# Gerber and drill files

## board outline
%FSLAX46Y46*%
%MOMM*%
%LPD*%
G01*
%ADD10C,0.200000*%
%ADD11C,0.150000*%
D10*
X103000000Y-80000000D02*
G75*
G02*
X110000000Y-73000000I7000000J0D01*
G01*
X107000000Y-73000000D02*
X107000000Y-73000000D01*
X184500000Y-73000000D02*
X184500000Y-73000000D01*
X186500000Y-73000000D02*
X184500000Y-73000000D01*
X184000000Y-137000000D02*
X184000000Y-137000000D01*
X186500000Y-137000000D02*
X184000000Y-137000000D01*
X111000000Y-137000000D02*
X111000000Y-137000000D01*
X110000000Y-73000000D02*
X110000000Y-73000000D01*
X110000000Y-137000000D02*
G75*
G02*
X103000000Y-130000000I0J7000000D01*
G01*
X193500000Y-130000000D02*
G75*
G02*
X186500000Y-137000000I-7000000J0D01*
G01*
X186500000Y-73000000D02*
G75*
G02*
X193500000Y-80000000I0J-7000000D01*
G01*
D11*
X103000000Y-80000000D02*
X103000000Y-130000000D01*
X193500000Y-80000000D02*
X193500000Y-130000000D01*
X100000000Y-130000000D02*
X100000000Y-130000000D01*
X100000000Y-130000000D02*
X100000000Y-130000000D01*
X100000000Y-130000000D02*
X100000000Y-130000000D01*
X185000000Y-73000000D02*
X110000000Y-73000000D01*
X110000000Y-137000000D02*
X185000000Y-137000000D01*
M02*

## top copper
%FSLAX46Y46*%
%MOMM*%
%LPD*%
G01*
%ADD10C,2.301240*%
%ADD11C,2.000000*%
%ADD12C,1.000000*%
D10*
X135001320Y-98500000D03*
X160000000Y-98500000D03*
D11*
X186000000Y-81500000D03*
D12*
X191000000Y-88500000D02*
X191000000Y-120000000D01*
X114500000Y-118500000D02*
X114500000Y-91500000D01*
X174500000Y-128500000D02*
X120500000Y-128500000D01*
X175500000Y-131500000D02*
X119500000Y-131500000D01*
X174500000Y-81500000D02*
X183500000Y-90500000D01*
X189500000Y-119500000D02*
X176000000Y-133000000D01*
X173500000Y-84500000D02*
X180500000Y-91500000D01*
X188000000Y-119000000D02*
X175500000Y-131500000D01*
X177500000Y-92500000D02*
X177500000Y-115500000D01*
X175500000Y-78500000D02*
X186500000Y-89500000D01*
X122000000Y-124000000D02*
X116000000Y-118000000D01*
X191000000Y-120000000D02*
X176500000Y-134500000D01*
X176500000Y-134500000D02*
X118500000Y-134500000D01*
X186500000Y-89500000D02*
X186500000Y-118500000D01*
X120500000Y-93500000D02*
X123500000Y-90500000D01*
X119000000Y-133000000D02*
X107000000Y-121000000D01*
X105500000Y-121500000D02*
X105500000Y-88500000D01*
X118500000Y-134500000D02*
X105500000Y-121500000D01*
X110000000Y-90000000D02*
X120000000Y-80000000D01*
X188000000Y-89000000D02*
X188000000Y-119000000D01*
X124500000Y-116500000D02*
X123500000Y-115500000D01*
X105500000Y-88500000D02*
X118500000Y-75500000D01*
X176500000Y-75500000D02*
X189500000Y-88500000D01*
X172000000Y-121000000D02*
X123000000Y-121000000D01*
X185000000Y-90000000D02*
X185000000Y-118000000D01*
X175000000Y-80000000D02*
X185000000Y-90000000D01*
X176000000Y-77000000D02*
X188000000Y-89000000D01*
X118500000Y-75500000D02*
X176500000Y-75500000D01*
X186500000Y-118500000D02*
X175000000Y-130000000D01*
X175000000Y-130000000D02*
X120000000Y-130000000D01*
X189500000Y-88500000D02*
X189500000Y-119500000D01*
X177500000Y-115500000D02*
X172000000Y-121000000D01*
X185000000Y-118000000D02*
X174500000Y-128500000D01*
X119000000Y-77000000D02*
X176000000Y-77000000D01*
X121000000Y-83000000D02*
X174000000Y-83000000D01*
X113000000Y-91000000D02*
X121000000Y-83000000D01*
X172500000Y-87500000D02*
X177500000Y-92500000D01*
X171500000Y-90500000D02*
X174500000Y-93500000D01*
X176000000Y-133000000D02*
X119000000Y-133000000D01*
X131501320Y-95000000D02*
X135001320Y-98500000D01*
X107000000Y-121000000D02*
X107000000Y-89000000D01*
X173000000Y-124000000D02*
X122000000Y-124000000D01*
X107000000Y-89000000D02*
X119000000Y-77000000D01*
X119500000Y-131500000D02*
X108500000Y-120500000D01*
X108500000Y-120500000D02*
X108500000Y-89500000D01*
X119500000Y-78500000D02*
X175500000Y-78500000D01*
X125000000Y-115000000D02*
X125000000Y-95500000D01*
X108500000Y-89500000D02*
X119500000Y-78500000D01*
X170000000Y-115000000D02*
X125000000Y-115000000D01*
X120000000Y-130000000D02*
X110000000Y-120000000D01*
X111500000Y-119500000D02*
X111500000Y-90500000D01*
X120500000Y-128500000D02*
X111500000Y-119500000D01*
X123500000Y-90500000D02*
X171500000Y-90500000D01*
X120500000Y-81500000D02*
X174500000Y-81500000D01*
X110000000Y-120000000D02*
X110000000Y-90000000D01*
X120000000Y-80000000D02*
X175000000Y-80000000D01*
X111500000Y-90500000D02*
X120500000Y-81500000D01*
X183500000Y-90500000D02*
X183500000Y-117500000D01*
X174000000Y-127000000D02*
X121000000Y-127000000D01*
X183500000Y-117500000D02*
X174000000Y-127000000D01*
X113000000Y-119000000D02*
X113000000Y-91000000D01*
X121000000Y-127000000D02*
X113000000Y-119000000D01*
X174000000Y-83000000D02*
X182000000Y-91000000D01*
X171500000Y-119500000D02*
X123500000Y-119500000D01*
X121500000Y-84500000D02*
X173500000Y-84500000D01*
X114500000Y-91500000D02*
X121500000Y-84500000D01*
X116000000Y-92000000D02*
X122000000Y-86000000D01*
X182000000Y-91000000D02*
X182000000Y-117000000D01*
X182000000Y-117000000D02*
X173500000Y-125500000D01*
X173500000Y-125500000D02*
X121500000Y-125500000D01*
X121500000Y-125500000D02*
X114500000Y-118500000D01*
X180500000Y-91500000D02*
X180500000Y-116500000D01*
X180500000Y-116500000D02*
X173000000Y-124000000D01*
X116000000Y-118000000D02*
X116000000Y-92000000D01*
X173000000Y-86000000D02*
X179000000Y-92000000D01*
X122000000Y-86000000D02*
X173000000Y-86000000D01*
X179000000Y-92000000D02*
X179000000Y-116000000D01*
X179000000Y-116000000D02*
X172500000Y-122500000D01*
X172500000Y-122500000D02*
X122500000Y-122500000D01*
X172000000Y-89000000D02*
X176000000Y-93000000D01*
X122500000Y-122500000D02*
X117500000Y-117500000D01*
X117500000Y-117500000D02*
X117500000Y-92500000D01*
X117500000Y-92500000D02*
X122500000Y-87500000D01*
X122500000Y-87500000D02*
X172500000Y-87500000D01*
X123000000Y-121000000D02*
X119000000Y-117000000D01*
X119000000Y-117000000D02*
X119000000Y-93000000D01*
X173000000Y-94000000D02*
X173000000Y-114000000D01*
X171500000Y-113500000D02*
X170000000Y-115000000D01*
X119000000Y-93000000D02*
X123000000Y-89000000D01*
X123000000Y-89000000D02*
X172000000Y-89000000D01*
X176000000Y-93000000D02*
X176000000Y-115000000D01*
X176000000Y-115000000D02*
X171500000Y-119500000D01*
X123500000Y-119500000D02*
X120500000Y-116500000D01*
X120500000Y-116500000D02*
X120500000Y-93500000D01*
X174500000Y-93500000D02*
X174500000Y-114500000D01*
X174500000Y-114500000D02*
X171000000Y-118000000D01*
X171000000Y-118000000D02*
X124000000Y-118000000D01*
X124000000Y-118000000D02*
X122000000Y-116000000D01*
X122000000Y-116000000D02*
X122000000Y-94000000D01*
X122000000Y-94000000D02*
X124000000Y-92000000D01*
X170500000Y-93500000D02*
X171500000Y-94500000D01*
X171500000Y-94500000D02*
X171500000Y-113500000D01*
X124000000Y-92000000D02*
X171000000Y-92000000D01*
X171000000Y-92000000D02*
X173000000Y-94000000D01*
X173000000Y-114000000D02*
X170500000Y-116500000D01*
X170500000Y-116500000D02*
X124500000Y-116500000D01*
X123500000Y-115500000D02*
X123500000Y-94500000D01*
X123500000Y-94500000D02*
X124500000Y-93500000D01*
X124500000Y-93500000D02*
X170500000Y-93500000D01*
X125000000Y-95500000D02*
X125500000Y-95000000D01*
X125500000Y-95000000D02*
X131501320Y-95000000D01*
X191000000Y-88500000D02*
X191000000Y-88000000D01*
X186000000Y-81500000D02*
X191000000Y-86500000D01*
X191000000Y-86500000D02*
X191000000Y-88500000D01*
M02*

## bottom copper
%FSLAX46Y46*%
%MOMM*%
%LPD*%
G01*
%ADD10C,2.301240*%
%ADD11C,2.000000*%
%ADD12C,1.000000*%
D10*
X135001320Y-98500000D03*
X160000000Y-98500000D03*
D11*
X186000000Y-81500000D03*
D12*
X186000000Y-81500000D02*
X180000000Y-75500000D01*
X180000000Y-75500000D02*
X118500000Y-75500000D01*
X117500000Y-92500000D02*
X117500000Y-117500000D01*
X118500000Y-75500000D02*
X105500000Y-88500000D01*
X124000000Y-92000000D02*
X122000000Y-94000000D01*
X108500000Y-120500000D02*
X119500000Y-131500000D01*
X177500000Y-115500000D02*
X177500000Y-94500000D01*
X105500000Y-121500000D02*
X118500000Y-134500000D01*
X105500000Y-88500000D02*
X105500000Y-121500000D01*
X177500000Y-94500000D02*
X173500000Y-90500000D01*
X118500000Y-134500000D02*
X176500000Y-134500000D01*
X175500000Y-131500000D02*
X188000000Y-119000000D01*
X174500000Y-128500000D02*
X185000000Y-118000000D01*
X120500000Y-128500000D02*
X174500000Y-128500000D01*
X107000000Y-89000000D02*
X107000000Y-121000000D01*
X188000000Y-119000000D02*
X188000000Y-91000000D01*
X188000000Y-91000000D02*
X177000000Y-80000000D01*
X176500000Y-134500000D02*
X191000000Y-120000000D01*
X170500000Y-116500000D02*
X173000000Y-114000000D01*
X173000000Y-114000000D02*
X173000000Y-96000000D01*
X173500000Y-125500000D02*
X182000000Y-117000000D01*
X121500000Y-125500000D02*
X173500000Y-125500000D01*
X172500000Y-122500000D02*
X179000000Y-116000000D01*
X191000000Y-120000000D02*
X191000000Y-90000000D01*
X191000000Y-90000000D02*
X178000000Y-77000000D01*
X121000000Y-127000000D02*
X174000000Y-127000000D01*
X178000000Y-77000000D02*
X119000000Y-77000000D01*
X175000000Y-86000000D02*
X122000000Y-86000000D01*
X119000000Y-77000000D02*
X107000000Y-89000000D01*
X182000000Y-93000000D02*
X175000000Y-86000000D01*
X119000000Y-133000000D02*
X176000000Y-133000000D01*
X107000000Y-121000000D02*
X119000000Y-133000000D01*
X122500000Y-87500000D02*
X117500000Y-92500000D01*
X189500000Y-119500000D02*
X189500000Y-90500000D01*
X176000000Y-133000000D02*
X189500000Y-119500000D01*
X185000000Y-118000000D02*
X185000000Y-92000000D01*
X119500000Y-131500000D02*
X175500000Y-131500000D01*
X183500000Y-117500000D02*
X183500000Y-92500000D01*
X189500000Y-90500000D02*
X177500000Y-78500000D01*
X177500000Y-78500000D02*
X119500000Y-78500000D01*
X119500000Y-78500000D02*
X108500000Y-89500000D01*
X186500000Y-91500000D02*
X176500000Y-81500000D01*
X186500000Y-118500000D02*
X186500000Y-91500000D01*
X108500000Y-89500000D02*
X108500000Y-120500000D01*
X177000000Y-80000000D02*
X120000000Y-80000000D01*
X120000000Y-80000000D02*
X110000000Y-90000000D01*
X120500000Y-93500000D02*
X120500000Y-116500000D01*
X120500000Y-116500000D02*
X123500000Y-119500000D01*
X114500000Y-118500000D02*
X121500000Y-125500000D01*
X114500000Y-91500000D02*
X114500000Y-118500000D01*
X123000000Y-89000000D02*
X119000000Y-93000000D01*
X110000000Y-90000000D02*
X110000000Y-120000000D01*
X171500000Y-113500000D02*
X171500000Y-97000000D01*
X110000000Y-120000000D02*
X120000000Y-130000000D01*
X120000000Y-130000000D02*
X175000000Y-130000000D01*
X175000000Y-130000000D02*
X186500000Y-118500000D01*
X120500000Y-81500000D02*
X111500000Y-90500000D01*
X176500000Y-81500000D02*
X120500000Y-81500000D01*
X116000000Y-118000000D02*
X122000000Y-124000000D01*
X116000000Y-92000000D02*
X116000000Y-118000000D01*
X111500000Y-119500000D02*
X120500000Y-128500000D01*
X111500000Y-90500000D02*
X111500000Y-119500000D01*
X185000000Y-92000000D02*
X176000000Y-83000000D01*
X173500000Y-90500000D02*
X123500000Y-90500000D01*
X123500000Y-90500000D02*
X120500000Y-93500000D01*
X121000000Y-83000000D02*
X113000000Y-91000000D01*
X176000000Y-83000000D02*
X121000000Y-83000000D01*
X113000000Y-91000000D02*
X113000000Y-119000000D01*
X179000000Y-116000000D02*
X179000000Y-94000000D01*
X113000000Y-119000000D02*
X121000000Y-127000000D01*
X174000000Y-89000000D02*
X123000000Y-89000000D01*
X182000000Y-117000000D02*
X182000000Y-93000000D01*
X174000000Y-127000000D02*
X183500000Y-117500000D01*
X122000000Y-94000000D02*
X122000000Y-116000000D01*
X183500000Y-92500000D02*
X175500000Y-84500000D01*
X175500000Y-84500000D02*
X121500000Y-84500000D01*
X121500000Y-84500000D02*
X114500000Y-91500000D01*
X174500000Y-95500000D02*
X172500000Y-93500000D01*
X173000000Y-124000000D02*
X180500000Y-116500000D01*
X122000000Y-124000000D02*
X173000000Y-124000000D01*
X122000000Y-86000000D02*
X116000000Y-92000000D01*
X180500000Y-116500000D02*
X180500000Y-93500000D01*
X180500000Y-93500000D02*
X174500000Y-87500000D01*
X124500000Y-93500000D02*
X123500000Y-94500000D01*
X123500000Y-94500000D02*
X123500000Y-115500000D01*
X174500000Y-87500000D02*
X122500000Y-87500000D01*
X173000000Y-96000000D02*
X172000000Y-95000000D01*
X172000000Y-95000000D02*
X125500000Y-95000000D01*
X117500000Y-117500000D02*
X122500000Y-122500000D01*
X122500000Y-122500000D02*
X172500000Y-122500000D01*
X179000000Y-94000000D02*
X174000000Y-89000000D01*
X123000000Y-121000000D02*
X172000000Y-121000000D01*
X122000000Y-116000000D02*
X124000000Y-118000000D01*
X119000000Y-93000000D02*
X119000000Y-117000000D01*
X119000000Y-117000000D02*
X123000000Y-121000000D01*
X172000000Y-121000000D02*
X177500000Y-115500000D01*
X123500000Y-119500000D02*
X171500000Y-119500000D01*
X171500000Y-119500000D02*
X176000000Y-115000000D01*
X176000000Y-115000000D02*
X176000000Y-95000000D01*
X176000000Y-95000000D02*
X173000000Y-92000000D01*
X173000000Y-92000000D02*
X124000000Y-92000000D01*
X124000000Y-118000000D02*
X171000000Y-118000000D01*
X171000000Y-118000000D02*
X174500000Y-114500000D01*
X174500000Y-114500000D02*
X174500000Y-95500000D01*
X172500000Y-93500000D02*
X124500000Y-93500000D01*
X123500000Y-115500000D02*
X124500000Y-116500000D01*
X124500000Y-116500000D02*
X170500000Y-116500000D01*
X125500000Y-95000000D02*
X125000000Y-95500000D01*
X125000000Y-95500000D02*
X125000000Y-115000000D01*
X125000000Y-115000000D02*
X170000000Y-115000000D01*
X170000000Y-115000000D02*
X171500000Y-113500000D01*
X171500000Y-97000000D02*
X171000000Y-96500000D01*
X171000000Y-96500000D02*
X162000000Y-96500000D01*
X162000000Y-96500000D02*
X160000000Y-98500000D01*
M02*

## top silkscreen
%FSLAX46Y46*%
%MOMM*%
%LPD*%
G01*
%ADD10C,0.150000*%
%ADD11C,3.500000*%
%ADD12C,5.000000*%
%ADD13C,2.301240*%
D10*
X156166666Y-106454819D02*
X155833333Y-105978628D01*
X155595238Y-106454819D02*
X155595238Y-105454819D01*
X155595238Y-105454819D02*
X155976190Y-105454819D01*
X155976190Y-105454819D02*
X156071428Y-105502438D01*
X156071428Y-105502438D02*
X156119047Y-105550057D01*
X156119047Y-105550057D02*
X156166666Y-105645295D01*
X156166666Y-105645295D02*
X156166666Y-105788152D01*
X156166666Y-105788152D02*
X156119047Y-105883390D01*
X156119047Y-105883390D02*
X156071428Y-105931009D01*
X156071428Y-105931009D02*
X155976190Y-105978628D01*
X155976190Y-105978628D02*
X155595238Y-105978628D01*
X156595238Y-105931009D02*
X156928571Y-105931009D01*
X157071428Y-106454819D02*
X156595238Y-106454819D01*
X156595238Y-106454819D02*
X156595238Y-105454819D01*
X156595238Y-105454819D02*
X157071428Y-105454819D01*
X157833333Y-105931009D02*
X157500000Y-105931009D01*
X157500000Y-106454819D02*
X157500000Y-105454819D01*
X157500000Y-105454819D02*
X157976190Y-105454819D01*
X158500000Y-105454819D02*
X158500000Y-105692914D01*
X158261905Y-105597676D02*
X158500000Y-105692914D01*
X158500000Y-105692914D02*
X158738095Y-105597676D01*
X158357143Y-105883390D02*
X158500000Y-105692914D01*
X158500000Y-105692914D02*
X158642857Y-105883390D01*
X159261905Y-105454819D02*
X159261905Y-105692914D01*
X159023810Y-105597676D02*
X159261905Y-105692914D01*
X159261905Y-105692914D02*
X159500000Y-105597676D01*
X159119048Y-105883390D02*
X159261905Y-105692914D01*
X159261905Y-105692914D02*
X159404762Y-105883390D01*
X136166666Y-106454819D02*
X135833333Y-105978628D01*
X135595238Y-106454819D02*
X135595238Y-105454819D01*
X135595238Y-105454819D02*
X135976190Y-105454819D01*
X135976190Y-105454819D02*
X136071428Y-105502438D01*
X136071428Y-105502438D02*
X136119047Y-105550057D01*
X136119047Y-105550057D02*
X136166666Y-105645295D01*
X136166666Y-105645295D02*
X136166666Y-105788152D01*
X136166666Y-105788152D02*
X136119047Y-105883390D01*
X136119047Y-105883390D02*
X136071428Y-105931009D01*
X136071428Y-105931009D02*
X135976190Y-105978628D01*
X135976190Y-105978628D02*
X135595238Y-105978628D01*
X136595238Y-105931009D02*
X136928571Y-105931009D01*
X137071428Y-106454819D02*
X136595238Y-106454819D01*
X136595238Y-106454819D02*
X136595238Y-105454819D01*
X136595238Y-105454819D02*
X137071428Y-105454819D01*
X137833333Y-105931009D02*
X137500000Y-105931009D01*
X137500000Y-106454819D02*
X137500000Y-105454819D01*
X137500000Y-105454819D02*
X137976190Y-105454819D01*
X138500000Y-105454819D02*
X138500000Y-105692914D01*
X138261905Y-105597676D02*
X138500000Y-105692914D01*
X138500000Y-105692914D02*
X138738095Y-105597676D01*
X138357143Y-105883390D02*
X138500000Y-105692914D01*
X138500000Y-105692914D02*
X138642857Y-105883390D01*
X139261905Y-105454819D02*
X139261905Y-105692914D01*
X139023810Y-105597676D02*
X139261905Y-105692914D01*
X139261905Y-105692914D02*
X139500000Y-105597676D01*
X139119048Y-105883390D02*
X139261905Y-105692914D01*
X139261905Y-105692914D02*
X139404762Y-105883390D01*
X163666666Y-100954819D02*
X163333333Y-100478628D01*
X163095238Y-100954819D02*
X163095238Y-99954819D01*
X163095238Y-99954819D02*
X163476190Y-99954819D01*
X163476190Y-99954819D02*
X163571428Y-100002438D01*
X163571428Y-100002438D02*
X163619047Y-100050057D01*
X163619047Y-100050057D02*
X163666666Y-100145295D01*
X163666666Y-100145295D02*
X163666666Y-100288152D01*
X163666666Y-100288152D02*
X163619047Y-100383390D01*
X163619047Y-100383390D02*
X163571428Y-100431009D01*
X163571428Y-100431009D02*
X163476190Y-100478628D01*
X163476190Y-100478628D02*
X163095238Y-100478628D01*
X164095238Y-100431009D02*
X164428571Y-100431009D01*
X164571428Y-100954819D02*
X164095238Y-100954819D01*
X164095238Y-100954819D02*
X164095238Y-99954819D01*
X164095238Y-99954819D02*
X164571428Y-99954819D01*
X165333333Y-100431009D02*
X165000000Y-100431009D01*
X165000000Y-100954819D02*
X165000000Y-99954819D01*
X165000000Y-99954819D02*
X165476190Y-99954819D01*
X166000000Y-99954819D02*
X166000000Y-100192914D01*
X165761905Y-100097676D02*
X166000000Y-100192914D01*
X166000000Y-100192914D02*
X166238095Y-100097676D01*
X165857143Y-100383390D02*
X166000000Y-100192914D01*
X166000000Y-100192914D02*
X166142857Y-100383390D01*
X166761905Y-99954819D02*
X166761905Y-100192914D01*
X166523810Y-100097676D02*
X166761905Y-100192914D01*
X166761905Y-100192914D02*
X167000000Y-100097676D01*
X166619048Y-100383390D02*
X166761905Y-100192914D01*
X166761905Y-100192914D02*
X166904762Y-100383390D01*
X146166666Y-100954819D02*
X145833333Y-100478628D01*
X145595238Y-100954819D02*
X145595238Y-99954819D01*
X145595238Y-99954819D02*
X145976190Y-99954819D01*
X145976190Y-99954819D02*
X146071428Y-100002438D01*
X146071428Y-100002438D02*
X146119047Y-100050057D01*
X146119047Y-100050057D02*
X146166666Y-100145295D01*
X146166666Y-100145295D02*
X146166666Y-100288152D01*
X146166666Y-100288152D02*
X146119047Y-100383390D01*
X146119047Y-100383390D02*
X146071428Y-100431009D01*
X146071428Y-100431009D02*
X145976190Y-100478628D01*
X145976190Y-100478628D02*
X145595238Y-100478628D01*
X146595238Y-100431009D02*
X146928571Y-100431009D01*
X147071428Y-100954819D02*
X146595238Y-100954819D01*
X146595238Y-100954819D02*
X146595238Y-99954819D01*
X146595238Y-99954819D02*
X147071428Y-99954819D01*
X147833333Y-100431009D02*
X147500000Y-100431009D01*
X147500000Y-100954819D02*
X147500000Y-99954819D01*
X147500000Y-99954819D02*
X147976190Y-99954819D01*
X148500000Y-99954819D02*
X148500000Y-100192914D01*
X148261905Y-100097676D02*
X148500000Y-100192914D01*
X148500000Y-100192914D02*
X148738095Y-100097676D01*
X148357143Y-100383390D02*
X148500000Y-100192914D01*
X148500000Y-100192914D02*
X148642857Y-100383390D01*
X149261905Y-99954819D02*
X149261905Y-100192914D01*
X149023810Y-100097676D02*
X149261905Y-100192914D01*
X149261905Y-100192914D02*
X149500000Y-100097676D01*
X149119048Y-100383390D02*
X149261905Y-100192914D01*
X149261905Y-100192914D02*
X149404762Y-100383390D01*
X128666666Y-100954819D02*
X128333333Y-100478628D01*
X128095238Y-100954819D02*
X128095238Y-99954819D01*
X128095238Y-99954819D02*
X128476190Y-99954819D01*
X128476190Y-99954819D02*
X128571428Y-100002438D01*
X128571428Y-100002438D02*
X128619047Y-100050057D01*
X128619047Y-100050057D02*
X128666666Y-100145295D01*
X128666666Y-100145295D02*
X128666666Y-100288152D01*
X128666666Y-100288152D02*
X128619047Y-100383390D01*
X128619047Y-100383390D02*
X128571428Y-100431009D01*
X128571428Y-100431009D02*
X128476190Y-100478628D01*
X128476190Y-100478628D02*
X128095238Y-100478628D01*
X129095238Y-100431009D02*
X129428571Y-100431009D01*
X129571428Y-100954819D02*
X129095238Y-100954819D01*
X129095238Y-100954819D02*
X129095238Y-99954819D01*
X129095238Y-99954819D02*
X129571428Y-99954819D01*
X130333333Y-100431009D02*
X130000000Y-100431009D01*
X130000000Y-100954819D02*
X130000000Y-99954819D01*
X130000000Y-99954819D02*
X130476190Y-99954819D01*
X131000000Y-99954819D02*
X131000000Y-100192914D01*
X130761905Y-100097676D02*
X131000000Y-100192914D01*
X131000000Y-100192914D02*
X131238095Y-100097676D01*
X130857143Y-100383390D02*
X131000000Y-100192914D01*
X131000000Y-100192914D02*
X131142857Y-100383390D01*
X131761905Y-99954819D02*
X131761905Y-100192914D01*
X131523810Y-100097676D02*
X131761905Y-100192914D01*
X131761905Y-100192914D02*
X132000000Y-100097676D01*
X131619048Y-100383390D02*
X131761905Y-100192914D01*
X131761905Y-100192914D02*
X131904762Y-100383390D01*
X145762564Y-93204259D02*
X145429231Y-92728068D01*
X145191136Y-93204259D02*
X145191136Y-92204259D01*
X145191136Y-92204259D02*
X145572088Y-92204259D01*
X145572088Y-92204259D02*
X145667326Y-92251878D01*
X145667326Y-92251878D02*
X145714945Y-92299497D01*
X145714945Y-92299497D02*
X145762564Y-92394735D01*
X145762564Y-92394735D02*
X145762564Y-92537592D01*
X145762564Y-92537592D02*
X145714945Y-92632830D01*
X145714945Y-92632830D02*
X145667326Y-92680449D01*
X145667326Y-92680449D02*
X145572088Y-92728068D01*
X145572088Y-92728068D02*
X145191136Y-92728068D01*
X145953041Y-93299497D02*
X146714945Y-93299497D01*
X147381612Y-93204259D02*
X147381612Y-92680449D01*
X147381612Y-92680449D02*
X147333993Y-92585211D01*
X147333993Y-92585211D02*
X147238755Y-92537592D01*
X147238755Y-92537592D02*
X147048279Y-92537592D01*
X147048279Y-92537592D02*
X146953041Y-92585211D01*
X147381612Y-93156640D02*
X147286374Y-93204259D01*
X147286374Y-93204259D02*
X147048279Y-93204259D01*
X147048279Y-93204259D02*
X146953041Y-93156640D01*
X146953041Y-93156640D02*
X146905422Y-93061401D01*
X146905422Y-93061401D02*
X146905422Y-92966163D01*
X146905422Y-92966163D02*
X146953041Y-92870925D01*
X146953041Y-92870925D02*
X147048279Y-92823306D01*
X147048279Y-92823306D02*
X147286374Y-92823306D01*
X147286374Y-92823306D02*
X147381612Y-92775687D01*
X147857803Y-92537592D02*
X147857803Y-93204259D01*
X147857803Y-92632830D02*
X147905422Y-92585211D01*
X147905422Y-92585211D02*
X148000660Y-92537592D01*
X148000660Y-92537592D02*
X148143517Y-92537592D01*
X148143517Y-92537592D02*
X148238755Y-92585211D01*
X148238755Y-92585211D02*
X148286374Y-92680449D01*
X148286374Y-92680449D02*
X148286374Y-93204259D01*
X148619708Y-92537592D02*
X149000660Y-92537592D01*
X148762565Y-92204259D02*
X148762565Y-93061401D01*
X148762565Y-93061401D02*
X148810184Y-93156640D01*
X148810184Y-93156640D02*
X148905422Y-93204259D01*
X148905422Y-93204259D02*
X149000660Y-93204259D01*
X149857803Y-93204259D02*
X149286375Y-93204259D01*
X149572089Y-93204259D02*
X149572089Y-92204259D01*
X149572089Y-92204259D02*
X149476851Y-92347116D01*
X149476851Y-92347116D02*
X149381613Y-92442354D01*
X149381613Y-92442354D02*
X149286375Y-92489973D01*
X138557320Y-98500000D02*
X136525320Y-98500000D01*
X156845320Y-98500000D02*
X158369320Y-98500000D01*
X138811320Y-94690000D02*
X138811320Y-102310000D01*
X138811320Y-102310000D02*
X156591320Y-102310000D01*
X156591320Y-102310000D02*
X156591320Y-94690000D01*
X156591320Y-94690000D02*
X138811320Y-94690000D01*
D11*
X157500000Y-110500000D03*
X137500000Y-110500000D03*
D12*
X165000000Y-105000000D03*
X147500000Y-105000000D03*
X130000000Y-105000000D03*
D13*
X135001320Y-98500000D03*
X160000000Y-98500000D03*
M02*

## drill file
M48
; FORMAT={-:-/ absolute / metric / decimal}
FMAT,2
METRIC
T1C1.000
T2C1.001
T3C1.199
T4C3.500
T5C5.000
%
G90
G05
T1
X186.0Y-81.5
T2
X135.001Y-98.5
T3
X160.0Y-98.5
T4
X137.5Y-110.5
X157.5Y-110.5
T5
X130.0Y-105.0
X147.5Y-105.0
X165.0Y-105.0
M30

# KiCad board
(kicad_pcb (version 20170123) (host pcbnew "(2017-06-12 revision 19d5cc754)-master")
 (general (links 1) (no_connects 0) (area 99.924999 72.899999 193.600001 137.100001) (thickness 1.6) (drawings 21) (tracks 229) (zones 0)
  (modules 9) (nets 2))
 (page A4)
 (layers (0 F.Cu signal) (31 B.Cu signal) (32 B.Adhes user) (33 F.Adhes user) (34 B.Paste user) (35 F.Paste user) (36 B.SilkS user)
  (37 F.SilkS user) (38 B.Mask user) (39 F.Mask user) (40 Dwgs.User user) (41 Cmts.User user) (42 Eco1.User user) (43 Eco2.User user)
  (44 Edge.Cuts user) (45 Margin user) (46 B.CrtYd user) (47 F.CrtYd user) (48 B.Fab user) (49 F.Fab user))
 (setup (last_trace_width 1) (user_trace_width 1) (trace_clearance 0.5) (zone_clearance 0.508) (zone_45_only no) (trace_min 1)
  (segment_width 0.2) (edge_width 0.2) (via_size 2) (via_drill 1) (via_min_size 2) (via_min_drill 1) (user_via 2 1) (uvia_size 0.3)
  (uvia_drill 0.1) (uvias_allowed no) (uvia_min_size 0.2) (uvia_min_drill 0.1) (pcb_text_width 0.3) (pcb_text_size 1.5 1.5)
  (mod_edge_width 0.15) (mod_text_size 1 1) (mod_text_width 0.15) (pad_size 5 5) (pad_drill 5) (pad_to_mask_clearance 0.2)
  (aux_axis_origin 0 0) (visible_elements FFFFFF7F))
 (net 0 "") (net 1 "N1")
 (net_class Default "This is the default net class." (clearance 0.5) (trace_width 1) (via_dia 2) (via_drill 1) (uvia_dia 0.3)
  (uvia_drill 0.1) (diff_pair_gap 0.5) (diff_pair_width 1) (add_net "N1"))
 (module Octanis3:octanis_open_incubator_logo (layer B.Cu) (at 182.5 104.5 180)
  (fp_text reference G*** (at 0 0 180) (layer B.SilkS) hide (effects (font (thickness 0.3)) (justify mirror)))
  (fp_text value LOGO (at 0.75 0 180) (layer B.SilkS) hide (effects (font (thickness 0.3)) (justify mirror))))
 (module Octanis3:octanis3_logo (layer B.Cu) (at 147 125)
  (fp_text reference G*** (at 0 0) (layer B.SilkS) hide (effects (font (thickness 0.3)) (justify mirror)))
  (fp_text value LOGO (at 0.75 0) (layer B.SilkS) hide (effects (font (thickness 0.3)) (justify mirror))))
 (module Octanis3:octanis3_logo (layer B.Cu) (at 147.5 84.5)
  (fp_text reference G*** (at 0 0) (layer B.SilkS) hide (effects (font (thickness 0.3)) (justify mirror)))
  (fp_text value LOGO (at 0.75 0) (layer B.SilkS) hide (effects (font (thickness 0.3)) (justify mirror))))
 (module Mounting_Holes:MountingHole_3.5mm (layer F.Cu) (at 157.5 110.5)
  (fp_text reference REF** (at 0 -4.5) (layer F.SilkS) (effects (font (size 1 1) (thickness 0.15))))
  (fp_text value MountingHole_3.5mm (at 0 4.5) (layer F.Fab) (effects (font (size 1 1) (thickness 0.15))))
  (pad 1 np_thru_hole circle (at 0 0) (size 3.5 3.5) (drill 3.5) (layers *.Cu *.Mask F.SilkS)))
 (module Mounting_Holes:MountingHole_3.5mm (layer F.Cu) (at 137.5 110.5)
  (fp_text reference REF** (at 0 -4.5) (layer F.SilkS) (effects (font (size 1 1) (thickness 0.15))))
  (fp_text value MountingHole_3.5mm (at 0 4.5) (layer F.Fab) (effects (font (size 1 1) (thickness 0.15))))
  (pad 1 np_thru_hole circle (at 0 0) (size 3.5 3.5) (drill 3.5) (layers *.Cu *.Mask F.SilkS)))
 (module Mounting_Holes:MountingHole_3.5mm (layer F.Cu) (at 165 105)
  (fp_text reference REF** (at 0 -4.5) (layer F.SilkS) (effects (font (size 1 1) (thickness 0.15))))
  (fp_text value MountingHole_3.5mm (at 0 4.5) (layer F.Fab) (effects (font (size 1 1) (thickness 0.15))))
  (pad "" np_thru_hole circle (at 0 0) (size 5 5) (drill 5) (layers *.Cu *.Mask F.SilkS)))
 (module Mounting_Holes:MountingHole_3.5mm (layer F.Cu) (at 147.5 105)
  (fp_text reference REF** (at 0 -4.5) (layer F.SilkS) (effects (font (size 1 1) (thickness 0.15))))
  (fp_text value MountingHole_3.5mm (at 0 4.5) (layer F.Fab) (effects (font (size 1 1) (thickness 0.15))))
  (pad "" np_thru_hole circle (at 0 0) (size 5 5) (drill 5) (layers *.Cu *.Mask F.SilkS)))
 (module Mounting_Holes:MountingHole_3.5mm (layer F.Cu) (at 130 105)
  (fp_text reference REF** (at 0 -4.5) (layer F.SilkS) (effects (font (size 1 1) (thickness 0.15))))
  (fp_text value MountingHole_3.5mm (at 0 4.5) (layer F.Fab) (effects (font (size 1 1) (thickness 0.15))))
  (pad "" np_thru_hole circle (at 0 0) (size 5 5) (drill 5) (layers *.Cu *.Mask F.SilkS)))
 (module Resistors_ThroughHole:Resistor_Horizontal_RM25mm (layer F.Cu) (at 135.00132 98.5)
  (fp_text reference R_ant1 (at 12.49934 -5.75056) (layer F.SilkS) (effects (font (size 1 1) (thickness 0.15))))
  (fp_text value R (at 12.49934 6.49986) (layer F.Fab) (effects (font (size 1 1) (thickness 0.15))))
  (fp_line (start 3.556 0) (end 1.524 0) (layer F.SilkS) (width 0.15))
  (fp_line (start 21.844 0) (end 23.368 0) (layer F.SilkS) (width 0.15))
  (fp_line (start 3.81 -3.81) (end 3.81 3.81) (layer F.SilkS) (width 0.15))
  (fp_line (start 3.81 3.81) (end 21.59 3.81) (layer F.SilkS) (width 0.15))
  (fp_line (start 21.59 3.81) (end 21.59 -3.81) (layer F.SilkS) (width 0.15))
  (fp_line (start 21.59 -3.81) (end 3.81 -3.81) (layer F.SilkS) (width 0.15))
  (pad 1 thru_hole circle (at 0 0) (size 2.30124 2.30124) (drill 1.00076) (layers *.Cu *.SilkS *.Mask) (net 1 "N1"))
  (pad 2 thru_hole circle (at 24.99868 0) (size 2.30124 2.30124) (drill 1.19888) (layers *.Cu *.SilkS *.Mask) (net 1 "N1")))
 (gr_arc (start 110 80) (end 103 80) (angle 90) (layer Edge.Cuts) (width 0.2))
 (gr_line (start 107 73) (end 107 73) (layer Edge.Cuts) (width 0.2))
 (gr_line (start 184.5 73) (end 184.5 73) (layer Edge.Cuts) (width 0.2))
 (gr_line (start 186.5 73) (end 184.5 73) (layer Edge.Cuts) (width 0.2))
 (gr_line (start 184 137) (end 184 137) (layer Edge.Cuts) (width 0.2))
 (gr_line (start 186.5 137) (end 184 137) (layer Edge.Cuts) (width 0.2))
 (gr_line (start 111 137) (end 111 137) (layer Edge.Cuts) (width 0.2))
 (gr_line (start 110 73) (end 110 73) (layer Edge.Cuts) (width 0.2))
 (gr_arc (start 110 130) (end 110 137) (angle 90) (layer Edge.Cuts) (width 0.2))
 (gr_arc (start 186.5 130) (end 193.5 130) (angle 90) (layer Edge.Cuts) (width 0.2))
 (gr_arc (start 186.5 80) (end 186.5 73) (angle 90) (layer Edge.Cuts) (width 0.2))
 (gr_line (start 103 80) (end 103 130) (layer Edge.Cuts) (width 0.15))
 (gr_line (start 193.5 80) (end 193.5 130) (layer Edge.Cuts) (width 0.15))
 (gr_line (start 100 130) (end 100 130) (layer Edge.Cuts) (width 0.15))
 (gr_line (start 100 130) (end 100 130) (layer Edge.Cuts) (width 0.15))
 (gr_line (start 100 130) (end 100 130) (layer Edge.Cuts) (width 0.15))
 (gr_line (start 185 73) (end 110 73) (layer Edge.Cuts) (width 0.15))
 (gr_line (start 110 137) (end 185 137) (layer Edge.Cuts) (width 0.15))
 (segment (start 191 88.5) (end 191 120) (width 1) (layer F.Cu) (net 1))
 (segment (start 114.5 118.5) (end 114.5 91.5) (width 1) (layer F.Cu) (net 1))
 (segment (start 174.5 128.5) (end 120.5 128.5) (width 1) (layer F.Cu) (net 1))
 (segment (start 175.5 131.5) (end 119.5 131.5) (width 1) (layer F.Cu) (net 1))
 (segment (start 174.5 81.5) (end 183.5 90.5) (width 1) (layer F.Cu) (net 1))
 (segment (start 189.5 119.5) (end 176 133) (width 1) (layer F.Cu) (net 1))
 (segment (start 173.5 84.5) (end 180.5 91.5) (width 1) (layer F.Cu) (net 1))
 (segment (start 188 119) (end 175.5 131.5) (width 1) (layer F.Cu) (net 1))
 (segment (start 177.5 92.5) (end 177.5 115.5) (width 1) (layer F.Cu) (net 1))
 (segment (start 175.5 78.5) (end 186.5 89.5) (width 1) (layer F.Cu) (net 1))
 (segment (start 122 124) (end 116 118) (width 1) (layer F.Cu) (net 1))
 (segment (start 191 120) (end 176.5 134.5) (width 1) (layer F.Cu) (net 1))
 (segment (start 176.5 134.5) (end 118.5 134.5) (width 1) (layer F.Cu) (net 1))
 (segment (start 186.5 89.5) (end 186.5 118.5) (width 1) (layer F.Cu) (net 1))
 (segment (start 120.5 93.5) (end 123.5 90.5) (width 1) (layer F.Cu) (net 1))
 (segment (start 119 133) (end 107 121) (width 1) (layer F.Cu) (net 1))
 (segment (start 105.5 121.5) (end 105.5 88.5) (width 1) (layer F.Cu) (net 1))
 (segment (start 118.5 134.5) (end 105.5 121.5) (width 1) (layer F.Cu) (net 1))
 (segment (start 110 90) (end 120 80) (width 1) (layer F.Cu) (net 1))
 (segment (start 188 89) (end 188 119) (width 1) (layer F.Cu) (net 1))
 (segment (start 124.5 116.5) (end 123.5 115.5) (width 1) (layer F.Cu) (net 1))
 (segment (start 105.5 88.5) (end 118.5 75.5) (width 1) (layer F.Cu) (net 1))
 (segment (start 176.5 75.5) (end 189.5 88.5) (width 1) (layer F.Cu) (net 1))
 (segment (start 172 121) (end 123 121) (width 1) (layer F.Cu) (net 1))
 (segment (start 185 90) (end 185 118) (width 1) (layer F.Cu) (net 1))
 (segment (start 175 80) (end 185 90) (width 1) (layer F.Cu) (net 1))
 (segment (start 176 77) (end 188 89) (width 1) (layer F.Cu) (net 1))
 (segment (start 118.5 75.5) (end 176.5 75.5) (width 1) (layer F.Cu) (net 1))
 (segment (start 186.5 118.5) (end 175 130) (width 1) (layer F.Cu) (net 1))
 (segment (start 175 130) (end 120 130) (width 1) (layer F.Cu) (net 1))
 (segment (start 189.5 88.5) (end 189.5 119.5) (width 1) (layer F.Cu) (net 1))
 (segment (start 177.5 115.5) (end 172 121) (width 1) (layer F.Cu) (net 1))
 (segment (start 185 118) (end 174.5 128.5) (width 1) (layer F.Cu) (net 1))
 (segment (start 119 77) (end 176 77) (width 1) (layer F.Cu) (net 1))
 (segment (start 121 83) (end 174 83) (width 1) (layer F.Cu) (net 1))
 (segment (start 113 91) (end 121 83) (width 1) (layer F.Cu) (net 1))
 (segment (start 172.5 87.5) (end 177.5 92.5) (width 1) (layer F.Cu) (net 1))
 (segment (start 171.5 90.5) (end 174.5 93.5) (width 1) (layer F.Cu) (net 1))
 (segment (start 176 133) (end 119 133) (width 1) (layer F.Cu) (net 1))
 (segment (start 131.50132 95) (end 135.00132 98.5) (width 1) (layer F.Cu) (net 1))
 (segment (start 107 121) (end 107 89) (width 1) (layer F.Cu) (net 1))
 (segment (start 173 124) (end 122 124) (width 1) (layer F.Cu) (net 1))
 (segment (start 107 89) (end 119 77) (width 1) (layer F.Cu) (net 1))
 (segment (start 119.5 131.5) (end 108.5 120.5) (width 1) (layer F.Cu) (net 1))
 (segment (start 108.5 120.5) (end 108.5 89.5) (width 1) (layer F.Cu) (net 1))
 (segment (start 119.5 78.5) (end 175.5 78.5) (width 1) (layer F.Cu) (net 1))
 (segment (start 125 115) (end 125 95.5) (width 1) (layer F.Cu) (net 1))
 (segment (start 108.5 89.5) (end 119.5 78.5) (width 1) (layer F.Cu) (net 1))
 (segment (start 170 115) (end 125 115) (width 1) (layer F.Cu) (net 1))
 (segment (start 120 130) (end 110 120) (width 1) (layer F.Cu) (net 1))
 (segment (start 111.5 119.5) (end 111.5 90.5) (width 1) (layer F.Cu) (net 1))
 (segment (start 120.5 128.5) (end 111.5 119.5) (width 1) (layer F.Cu) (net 1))
 (segment (start 123.5 90.5) (end 171.5 90.5) (width 1) (layer F.Cu) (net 1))
 (segment (start 120.5 81.5) (end 174.5 81.5) (width 1) (layer F.Cu) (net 1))
 (segment (start 110 120) (end 110 90) (width 1) (layer F.Cu) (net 1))
 (segment (start 120 80) (end 175 80) (width 1) (layer F.Cu) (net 1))
 (segment (start 111.5 90.5) (end 120.5 81.5) (width 1) (layer F.Cu) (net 1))
 (segment (start 183.5 90.5) (end 183.5 117.5) (width 1) (layer F.Cu) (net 1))
 (segment (start 174 127) (end 121 127) (width 1) (layer F.Cu) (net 1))
 (segment (start 183.5 117.5) (end 174 127) (width 1) (layer F.Cu) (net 1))
 (segment (start 113 119) (end 113 91) (width 1) (layer F.Cu) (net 1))
 (segment (start 121 127) (end 113 119) (width 1) (layer F.Cu) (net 1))
 (segment (start 174 83) (end 182 91) (width 1) (layer F.Cu) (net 1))
 (segment (start 171.5 119.5) (end 123.5 119.5) (width 1) (layer F.Cu) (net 1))
 (segment (start 121.5 84.5) (end 173.5 84.5) (width 1) (layer F.Cu) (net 1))
 (segment (start 114.5 91.5) (end 121.5 84.5) (width 1) (layer F.Cu) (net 1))
 (segment (start 116 92) (end 122 86) (width 1) (layer F.Cu) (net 1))
 (segment (start 182 91) (end 182 117) (width 1) (layer F.Cu) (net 1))
 (segment (start 182 117) (end 173.5 125.5) (width 1) (layer F.Cu) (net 1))
 (segment (start 173.5 125.5) (end 121.5 125.5) (width 1) (layer F.Cu) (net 1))
 (segment (start 121.5 125.5) (end 114.5 118.5) (width 1) (layer F.Cu) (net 1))
 (segment (start 180.5 91.5) (end 180.5 116.5) (width 1) (layer F.Cu) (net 1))
 (segment (start 180.5 116.5) (end 173 124) (width 1) (layer F.Cu) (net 1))
 (segment (start 116 118) (end 116 92) (width 1) (layer F.Cu) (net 1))
 (segment (start 173 86) (end 179 92) (width 1) (layer F.Cu) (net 1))
 (segment (start 122 86) (end 173 86) (width 1) (layer F.Cu) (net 1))
 (segment (start 179 92) (end 179 116) (width 1) (layer F.Cu) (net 1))
 (segment (start 179 116) (end 172.5 122.5) (width 1) (layer F.Cu) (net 1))
 (segment (start 172.5 122.5) (end 122.5 122.5) (width 1) (layer F.Cu) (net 1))
 (segment (start 172 89) (end 176 93) (width 1) (layer F.Cu) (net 1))
 (segment (start 122.5 122.5) (end 117.5 117.5) (width 1) (layer F.Cu) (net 1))
 (segment (start 117.5 117.5) (end 117.5 92.5) (width 1) (layer F.Cu) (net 1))
 (segment (start 117.5 92.5) (end 122.5 87.5) (width 1) (layer F.Cu) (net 1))
 (segment (start 122.5 87.5) (end 172.5 87.5) (width 1) (layer F.Cu) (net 1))
 (segment (start 123 121) (end 119 117) (width 1) (layer F.Cu) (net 1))
 (segment (start 119 117) (end 119 93) (width 1) (layer F.Cu) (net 1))
 (segment (start 173 94) (end 173 114) (width 1) (layer F.Cu) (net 1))
 (segment (start 171.5 113.5) (end 170 115) (width 1) (layer F.Cu) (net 1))
 (segment (start 119 93) (end 123 89) (width 1) (layer F.Cu) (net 1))
 (segment (start 123 89) (end 172 89) (width 1) (layer F.Cu) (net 1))
 (segment (start 176 93) (end 176 115) (width 1) (layer F.Cu) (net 1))
 (segment (start 176 115) (end 171.5 119.5) (width 1) (layer F.Cu) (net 1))
 (segment (start 123.5 119.5) (end 120.5 116.5) (width 1) (layer F.Cu) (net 1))
 (segment (start 120.5 116.5) (end 120.5 93.5) (width 1) (layer F.Cu) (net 1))
 (segment (start 174.5 93.5) (end 174.5 114.5) (width 1) (layer F.Cu) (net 1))
 (segment (start 174.5 114.5) (end 171 118) (width 1) (layer F.Cu) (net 1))
 (segment (start 171 118) (end 124 118) (width 1) (layer F.Cu) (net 1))
 (segment (start 124 118) (end 122 116) (width 1) (layer F.Cu) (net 1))
 (segment (start 122 116) (end 122 94) (width 1) (layer F.Cu) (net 1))
 (segment (start 122 94) (end 124 92) (width 1) (layer F.Cu) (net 1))
 (segment (start 170.5 93.5) (end 171.5 94.5) (width 1) (layer F.Cu) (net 1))
 (segment (start 171.5 94.5) (end 171.5 113.5) (width 1) (layer F.Cu) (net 1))
 (segment (start 124 92) (end 171 92) (width 1) (layer F.Cu) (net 1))
 (segment (start 171 92) (end 173 94) (width 1) (layer F.Cu) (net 1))
 (segment (start 173 114) (end 170.5 116.5) (width 1) (layer F.Cu) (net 1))
 (segment (start 170.5 116.5) (end 124.5 116.5) (width 1) (layer F.Cu) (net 1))
 (segment (start 123.5 115.5) (end 123.5 94.5) (width 1) (layer F.Cu) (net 1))
 (segment (start 123.5 94.5) (end 124.5 93.5) (width 1) (layer F.Cu) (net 1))
 (segment (start 124.5 93.5) (end 170.5 93.5) (width 1) (layer F.Cu) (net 1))
 (segment (start 125 95.5) (end 125.5 95) (width 1) (layer F.Cu) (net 1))
 (segment (start 125.5 95) (end 131.50132 95) (width 1) (layer F.Cu) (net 1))
 (segment (start 186 81.5) (end 180 75.5) (width 1) (layer B.Cu) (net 1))
 (segment (start 180 75.5) (end 118.5 75.5) (width 1) (layer B.Cu) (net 1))
 (segment (start 117.5 92.5) (end 117.5 117.5) (width 1) (layer B.Cu) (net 1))
 (segment (start 118.5 75.5) (end 105.5 88.5) (width 1) (layer B.Cu) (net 1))
 (segment (start 124 92) (end 122 94) (width 1) (layer B.Cu) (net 1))
 (segment (start 108.5 120.5) (end 119.5 131.5) (width 1) (layer B.Cu) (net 1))
 (segment (start 177.5 115.5) (end 177.5 94.5) (width 1) (layer B.Cu) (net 1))
 (segment (start 105.5 121.5) (end 118.5 134.5) (width 1) (layer B.Cu) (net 1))
 (segment (start 105.5 88.5) (end 105.5 121.5) (width 1) (layer B.Cu) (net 1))
 (segment (start 177.5 94.5) (end 173.5 90.5) (width 1) (layer B.Cu) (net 1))
 (segment (start 118.5 134.5) (end 176.5 134.5) (width 1) (layer B.Cu) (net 1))
 (segment (start 175.5 131.5) (end 188 119) (width 1) (layer B.Cu) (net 1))
 (segment (start 174.5 128.5) (end 185 118) (width 1) (layer B.Cu) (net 1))
 (segment (start 120.5 128.5) (end 174.5 128.5) (width 1) (layer B.Cu) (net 1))
 (segment (start 107 89) (end 107 121) (width 1) (layer B.Cu) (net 1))
 (segment (start 188 119) (end 188 91) (width 1) (layer B.Cu) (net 1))
 (segment (start 188 91) (end 177 80) (width 1) (layer B.Cu) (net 1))
 (segment (start 176.5 134.5) (end 191 120) (width 1) (layer B.Cu) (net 1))
 (segment (start 170.5 116.5) (end 173 114) (width 1) (layer B.Cu) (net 1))
 (segment (start 173 114) (end 173 96) (width 1) (layer B.Cu) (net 1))
 (segment (start 173.5 125.5) (end 182 117) (width 1) (layer B.Cu) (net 1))
 (segment (start 121.5 125.5) (end 173.5 125.5) (width 1) (layer B.Cu) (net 1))
 (segment (start 172.5 122.5) (end 179 116) (width 1) (layer B.Cu) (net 1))
 (segment (start 191 120) (end 191 90) (width 1) (layer B.Cu) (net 1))
 (segment (start 191 90) (end 178 77) (width 1) (layer B.Cu) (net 1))
 (segment (start 121 127) (end 174 127) (width 1) (layer B.Cu) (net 1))
 (segment (start 178 77) (end 119 77) (width 1) (layer B.Cu) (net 1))
 (segment (start 175 86) (end 122 86) (width 1) (layer B.Cu) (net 1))
 (segment (start 119 77) (end 107 89) (width 1) (layer B.Cu) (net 1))
 (segment (start 182 93) (end 175 86) (width 1) (layer B.Cu) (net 1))
 (segment (start 119 133) (end 176 133) (width 1) (layer B.Cu) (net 1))
 (segment (start 107 121) (end 119 133) (width 1) (layer B.Cu) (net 1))
 (segment (start 122.5 87.5) (end 117.5 92.5) (width 1) (layer B.Cu) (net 1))
 (segment (start 189.5 119.5) (end 189.5 90.5) (width 1) (layer B.Cu) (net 1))
 (segment (start 176 133) (end 189.5 119.5) (width 1) (layer B.Cu) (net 1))
 (segment (start 185 118) (end 185 92) (width 1) (layer B.Cu) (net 1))
 (segment (start 119.5 131.5) (end 175.5 131.5) (width 1) (layer B.Cu) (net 1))
 (segment (start 183.5 117.5) (end 183.5 92.5) (width 1) (layer B.Cu) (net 1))
 (segment (start 189.5 90.5) (end 177.5 78.5) (width 1) (layer B.Cu) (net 1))
 (segment (start 177.5 78.5) (end 119.5 78.5) (width 1) (layer B.Cu) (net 1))
 (segment (start 119.5 78.5) (end 108.5 89.5) (width 1) (layer B.Cu) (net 1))
 (segment (start 186.5 91.5) (end 176.5 81.5) (width 1) (layer B.Cu) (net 1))
 (segment (start 186.5 118.5) (end 186.5 91.5) (width 1) (layer B.Cu) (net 1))
 (segment (start 108.5 89.5) (end 108.5 120.5) (width 1) (layer B.Cu) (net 1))
 (segment (start 177 80) (end 120 80) (width 1) (layer B.Cu) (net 1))
 (segment (start 120 80) (end 110 90) (width 1) (layer B.Cu) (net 1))
 (segment (start 120.5 93.5) (end 120.5 116.5) (width 1) (layer B.Cu) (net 1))
 (segment (start 120.5 116.5) (end 123.5 119.5) (width 1) (layer B.Cu) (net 1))
 (segment (start 114.5 118.5) (end 121.5 125.5) (width 1) (layer B.Cu) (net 1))
 (segment (start 114.5 91.5) (end 114.5 118.5) (width 1) (layer B.Cu) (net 1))
 (segment (start 123 89) (end 119 93) (width 1) (layer B.Cu) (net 1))
 (segment (start 110 90) (end 110 120) (width 1) (layer B.Cu) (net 1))
 (segment (start 171.5 113.5) (end 171.5 97) (width 1) (layer B.Cu) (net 1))
 (segment (start 110 120) (end 120 130) (width 1) (layer B.Cu) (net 1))
 (segment (start 120 130) (end 175 130) (width 1) (layer B.Cu) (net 1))
 (segment (start 175 130) (end 186.5 118.5) (width 1) (layer B.Cu) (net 1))
 (segment (start 120.5 81.5) (end 111.5 90.5) (width 1) (layer B.Cu) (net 1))
 (segment (start 176.5 81.5) (end 120.5 81.5) (width 1) (layer B.Cu) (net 1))
 (segment (start 116 118) (end 122 124) (width 1) (layer B.Cu) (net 1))
 (segment (start 116 92) (end 116 118) (width 1) (layer B.Cu) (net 1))
 (segment (start 111.5 119.5) (end 120.5 128.5) (width 1) (layer B.Cu) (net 1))
 (segment (start 111.5 90.5) (end 111.5 119.5) (width 1) (layer B.Cu) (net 1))
 (segment (start 185 92) (end 176 83) (width 1) (layer B.Cu) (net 1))
 (segment (start 173.5 90.5) (end 123.5 90.5) (width 1) (layer B.Cu) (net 1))
 (segment (start 123.5 90.5) (end 120.5 93.5) (width 1) (layer B.Cu) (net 1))
 (segment (start 121 83) (end 113 91) (width 1) (layer B.Cu) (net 1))
 (segment (start 176 83) (end 121 83) (width 1) (layer B.Cu) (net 1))
 (segment (start 113 91) (end 113 119) (width 1) (layer B.Cu) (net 1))
 (segment (start 179 116) (end 179 94) (width 1) (layer B.Cu) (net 1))
 (segment (start 113 119) (end 121 127) (width 1) (layer B.Cu) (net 1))
 (segment (start 174 89) (end 123 89) (width 1) (layer B.Cu) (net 1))
 (segment (start 182 117) (end 182 93) (width 1) (layer B.Cu) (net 1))
 (segment (start 174 127) (end 183.5 117.5) (width 1) (layer B.Cu) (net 1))
 (segment (start 122 94) (end 122 116) (width 1) (layer B.Cu) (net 1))
 (segment (start 183.5 92.5) (end 175.5 84.5) (width 1) (layer B.Cu) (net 1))
 (segment (start 175.5 84.5) (end 121.5 84.5) (width 1) (layer B.Cu) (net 1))
 (segment (start 121.5 84.5) (end 114.5 91.5) (width 1) (layer B.Cu) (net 1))
 (segment (start 174.5 95.5) (end 172.5 93.5) (width 1) (layer B.Cu) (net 1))
 (segment (start 173 124) (end 180.5 116.5) (width 1) (layer B.Cu) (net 1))
 (segment (start 122 124) (end 173 124) (width 1) (layer B.Cu) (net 1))
 (segment (start 122 86) (end 116 92) (width 1) (layer B.Cu) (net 1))
 (segment (start 180.5 116.5) (end 180.5 93.5) (width 1) (layer B.Cu) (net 1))
 (segment (start 180.5 93.5) (end 174.5 87.5) (width 1) (layer B.Cu) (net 1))
 (segment (start 124.5 93.5) (end 123.5 94.5) (width 1) (layer B.Cu) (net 1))
 (segment (start 123.5 94.5) (end 123.5 115.5) (width 1) (layer B.Cu) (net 1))
 (segment (start 174.5 87.5) (end 122.5 87.5) (width 1) (layer B.Cu) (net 1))
 (segment (start 173 96) (end 172 95) (width 1) (layer B.Cu) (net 1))
 (segment (start 172 95) (end 125.5 95) (width 1) (layer B.Cu) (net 1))
 (segment (start 117.5 117.5) (end 122.5 122.5) (width 1) (layer B.Cu) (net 1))
 (segment (start 122.5 122.5) (end 172.5 122.5) (width 1) (layer B.Cu) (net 1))
 (segment (start 179 94) (end 174 89) (width 1) (layer B.Cu) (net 1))
 (segment (start 123 121) (end 172 121) (width 1) (layer B.Cu) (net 1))
 (segment (start 122 116) (end 124 118) (width 1) (layer B.Cu) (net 1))
 (segment (start 119 93) (end 119 117) (width 1) (layer B.Cu) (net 1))
 (segment (start 119 117) (end 123 121) (width 1) (layer B.Cu) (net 1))
 (segment (start 172 121) (end 177.5 115.5) (width 1) (layer B.Cu) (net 1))
 (segment (start 123.5 119.5) (end 171.5 119.5) (width 1) (layer B.Cu) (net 1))
 (segment (start 171.5 119.5) (end 176 115) (width 1) (layer B.Cu) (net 1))
 (segment (start 176 115) (end 176 95) (width 1) (layer B.Cu) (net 1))
 (segment (start 176 95) (end 173 92) (width 1) (layer B.Cu) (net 1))
 (segment (start 173 92) (end 124 92) (width 1) (layer B.Cu) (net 1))
 (segment (start 124 118) (end 171 118) (width 1) (layer B.Cu) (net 1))
 (segment (start 171 118) (end 174.5 114.5) (width 1) (layer B.Cu) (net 1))
 (segment (start 174.5 114.5) (end 174.5 95.5) (width 1) (layer B.Cu) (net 1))
 (segment (start 172.5 93.5) (end 124.5 93.5) (width 1) (layer B.Cu) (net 1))
 (segment (start 123.5 115.5) (end 124.5 116.5) (width 1) (layer B.Cu) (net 1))
 (segment (start 124.5 116.5) (end 170.5 116.5) (width 1) (layer B.Cu) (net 1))
 (segment (start 125.5 95) (end 125 95.5) (width 1) (layer B.Cu) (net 1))
 (segment (start 125 95.5) (end 125 115) (width 1) (layer B.Cu) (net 1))
 (segment (start 125 115) (end 170 115) (width 1) (layer B.Cu) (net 1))
 (segment (start 170 115) (end 171.5 113.5) (width 1) (layer B.Cu) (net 1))
 (segment (start 171.5 97) (end 171 96.5) (width 1) (layer B.Cu) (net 1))
 (segment (start 171 96.5) (end 162 96.5) (width 1) (layer B.Cu) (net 1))
 (segment (start 162 96.5) (end 160 98.5) (width 1) (layer B.Cu) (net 1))
 (segment (start 191 88.5) (end 191 88) (width 1) (layer F.Cu) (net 1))
 (segment (start 186 81.5) (end 191 86.5) (width 1) (layer F.Cu) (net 1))
 (segment (start 191 86.5) (end 191 88.5) (width 1) (layer F.Cu) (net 1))
 (via (at 186 81.5) (size 2) (drill 1) (layers F.Cu B.Cu) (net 1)))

